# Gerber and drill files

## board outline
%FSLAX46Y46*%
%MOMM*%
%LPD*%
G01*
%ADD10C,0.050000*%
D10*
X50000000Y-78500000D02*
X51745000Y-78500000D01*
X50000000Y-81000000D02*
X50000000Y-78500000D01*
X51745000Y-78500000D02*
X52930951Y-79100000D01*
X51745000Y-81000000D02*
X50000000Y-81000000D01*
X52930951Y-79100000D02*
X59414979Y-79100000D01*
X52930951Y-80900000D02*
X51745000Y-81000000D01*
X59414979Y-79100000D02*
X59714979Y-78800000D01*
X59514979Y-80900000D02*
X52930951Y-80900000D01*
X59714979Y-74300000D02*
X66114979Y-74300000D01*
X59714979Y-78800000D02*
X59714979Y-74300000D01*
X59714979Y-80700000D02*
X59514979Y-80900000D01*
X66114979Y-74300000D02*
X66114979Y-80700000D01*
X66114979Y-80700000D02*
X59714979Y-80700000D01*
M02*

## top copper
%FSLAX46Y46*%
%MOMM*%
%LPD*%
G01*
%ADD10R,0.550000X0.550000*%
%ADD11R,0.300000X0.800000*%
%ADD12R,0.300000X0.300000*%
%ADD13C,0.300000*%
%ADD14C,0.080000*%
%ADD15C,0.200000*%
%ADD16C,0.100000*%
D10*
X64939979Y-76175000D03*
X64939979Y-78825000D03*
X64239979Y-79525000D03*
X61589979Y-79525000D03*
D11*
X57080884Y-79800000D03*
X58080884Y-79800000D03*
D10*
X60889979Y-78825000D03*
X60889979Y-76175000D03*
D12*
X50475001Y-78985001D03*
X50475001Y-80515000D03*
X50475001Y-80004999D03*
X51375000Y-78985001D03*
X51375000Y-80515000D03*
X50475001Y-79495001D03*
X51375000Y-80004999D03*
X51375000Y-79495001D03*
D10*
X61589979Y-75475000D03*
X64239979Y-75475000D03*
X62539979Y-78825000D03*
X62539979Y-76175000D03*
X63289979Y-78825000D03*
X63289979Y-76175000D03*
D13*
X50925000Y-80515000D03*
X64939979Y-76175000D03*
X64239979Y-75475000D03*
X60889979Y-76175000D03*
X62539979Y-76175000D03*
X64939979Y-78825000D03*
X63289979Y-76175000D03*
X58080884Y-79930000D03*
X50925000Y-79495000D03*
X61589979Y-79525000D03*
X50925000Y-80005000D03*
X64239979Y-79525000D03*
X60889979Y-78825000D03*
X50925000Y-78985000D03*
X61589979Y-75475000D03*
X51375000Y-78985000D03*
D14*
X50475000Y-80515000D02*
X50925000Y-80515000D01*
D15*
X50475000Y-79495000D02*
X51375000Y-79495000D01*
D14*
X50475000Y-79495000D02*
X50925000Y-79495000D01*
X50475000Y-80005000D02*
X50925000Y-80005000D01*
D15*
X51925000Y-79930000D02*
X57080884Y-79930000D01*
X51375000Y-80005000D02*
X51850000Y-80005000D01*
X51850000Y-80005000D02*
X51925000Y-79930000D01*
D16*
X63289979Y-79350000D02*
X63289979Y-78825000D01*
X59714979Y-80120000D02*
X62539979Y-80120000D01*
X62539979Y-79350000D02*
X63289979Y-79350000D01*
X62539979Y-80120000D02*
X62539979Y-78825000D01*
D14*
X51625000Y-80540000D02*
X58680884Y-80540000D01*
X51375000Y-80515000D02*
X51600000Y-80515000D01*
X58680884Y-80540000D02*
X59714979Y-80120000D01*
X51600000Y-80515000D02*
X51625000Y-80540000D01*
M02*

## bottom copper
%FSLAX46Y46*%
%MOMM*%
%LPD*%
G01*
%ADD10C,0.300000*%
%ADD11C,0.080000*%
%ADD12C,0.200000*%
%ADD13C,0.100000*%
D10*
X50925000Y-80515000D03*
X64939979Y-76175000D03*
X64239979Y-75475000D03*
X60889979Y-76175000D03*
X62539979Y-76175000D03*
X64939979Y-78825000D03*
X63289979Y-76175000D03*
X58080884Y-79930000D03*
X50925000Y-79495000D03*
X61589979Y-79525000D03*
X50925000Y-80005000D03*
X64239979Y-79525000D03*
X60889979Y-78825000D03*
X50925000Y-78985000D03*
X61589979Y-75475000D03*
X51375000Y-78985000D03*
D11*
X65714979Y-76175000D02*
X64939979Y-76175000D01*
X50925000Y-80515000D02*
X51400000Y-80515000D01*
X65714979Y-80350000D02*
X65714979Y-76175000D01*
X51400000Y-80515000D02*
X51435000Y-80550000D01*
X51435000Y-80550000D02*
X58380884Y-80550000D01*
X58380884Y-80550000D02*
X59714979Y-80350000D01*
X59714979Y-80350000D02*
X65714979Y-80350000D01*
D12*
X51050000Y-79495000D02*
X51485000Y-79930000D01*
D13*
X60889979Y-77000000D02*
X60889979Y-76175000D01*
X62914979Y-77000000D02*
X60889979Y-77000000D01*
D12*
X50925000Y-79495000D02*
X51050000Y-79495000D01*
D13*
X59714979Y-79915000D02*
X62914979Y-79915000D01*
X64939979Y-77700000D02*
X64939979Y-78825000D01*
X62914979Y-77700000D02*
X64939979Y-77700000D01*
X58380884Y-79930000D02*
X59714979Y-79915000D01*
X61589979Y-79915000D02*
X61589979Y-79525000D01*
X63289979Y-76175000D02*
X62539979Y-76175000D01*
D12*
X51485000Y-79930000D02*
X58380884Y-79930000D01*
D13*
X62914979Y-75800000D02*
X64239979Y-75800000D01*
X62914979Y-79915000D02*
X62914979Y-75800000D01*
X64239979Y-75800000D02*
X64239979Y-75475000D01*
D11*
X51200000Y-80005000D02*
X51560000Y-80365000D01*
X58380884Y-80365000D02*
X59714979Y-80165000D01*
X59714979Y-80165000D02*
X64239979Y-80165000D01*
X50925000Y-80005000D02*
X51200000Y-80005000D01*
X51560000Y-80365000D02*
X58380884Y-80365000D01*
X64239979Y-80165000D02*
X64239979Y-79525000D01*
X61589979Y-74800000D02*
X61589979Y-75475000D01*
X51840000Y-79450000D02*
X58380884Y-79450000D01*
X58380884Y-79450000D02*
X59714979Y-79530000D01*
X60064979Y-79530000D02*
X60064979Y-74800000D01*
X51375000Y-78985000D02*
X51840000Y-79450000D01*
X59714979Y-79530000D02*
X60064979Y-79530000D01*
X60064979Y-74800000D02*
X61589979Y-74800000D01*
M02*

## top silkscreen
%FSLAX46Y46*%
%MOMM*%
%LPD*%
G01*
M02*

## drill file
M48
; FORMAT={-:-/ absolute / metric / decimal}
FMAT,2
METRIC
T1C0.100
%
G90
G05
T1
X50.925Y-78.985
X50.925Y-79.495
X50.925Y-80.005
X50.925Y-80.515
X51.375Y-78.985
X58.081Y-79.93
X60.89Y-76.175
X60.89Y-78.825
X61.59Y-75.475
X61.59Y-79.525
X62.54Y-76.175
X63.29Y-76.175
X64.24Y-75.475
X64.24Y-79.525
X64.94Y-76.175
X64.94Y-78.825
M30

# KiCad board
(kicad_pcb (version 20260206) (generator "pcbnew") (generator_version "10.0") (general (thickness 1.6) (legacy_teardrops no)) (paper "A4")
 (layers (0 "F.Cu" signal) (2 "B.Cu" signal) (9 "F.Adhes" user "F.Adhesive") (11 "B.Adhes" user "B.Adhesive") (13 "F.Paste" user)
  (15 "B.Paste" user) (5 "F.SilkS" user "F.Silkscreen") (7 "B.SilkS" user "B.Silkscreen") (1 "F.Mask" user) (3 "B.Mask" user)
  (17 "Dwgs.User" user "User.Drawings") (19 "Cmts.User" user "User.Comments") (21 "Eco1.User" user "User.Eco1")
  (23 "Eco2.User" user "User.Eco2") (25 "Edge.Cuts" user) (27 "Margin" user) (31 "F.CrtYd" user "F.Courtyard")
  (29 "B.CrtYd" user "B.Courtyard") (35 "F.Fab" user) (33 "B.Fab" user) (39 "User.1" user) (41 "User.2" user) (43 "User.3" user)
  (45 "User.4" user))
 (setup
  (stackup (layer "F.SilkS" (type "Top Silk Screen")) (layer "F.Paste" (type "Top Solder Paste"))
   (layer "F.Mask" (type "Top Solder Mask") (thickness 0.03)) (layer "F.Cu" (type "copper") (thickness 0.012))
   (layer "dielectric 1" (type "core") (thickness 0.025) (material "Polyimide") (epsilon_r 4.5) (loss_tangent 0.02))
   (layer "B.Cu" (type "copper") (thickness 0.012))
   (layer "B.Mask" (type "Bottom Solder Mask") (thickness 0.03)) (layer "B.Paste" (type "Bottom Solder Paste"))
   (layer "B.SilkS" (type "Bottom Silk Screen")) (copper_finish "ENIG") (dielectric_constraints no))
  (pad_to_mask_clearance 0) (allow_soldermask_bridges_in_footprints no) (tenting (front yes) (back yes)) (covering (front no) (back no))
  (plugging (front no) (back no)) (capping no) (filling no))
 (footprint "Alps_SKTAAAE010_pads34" (layer "F.Cu") (at 65.314979 77.5 -90)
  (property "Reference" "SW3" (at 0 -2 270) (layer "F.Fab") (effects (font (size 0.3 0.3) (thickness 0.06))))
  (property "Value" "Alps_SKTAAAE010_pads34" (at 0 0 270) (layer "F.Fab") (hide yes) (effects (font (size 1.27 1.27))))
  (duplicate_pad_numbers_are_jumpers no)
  (pad "3" smd rect (at -1.325 0.375 270) (size 0.55 0.55) (layers "F.Cu" "F.Mask") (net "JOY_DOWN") (solder_mask_margin 0.05)
   (thermal_bridge_angle 45))
  (pad "4" smd rect (at 1.325 0.375 270) (size 0.55 0.55) (layers "F.Cu" "F.Mask") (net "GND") (solder_mask_margin 0.05)
   (thermal_bridge_angle 45)))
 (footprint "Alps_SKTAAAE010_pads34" (layer "F.Cu") (at 62.914979 79.9 180)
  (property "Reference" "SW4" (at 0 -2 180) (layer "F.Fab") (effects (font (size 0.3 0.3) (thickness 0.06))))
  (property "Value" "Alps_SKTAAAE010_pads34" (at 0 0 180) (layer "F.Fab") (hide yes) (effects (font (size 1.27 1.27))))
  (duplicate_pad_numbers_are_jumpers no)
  (pad "3" smd rect (at -1.325 0.375 180) (size 0.55 0.55) (layers "F.Cu" "F.Mask") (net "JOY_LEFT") (solder_mask_margin 0.05)
   (thermal_bridge_angle 45))
  (pad "4" smd rect (at 1.325 0.375 180) (size 0.55 0.55) (layers "F.Cu" "F.Mask") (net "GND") (solder_mask_margin 0.05)
   (thermal_bridge_angle 45)))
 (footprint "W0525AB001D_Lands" (layer "F.Cu") (at 57.580884 79.93)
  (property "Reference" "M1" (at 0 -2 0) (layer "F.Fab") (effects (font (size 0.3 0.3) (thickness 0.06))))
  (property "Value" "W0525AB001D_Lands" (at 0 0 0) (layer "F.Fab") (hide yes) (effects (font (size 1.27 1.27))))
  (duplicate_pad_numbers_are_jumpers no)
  (pad "1" smd rect (at -0.5 -0.13) (size 0.3 0.8) (layers "F.Cu" "F.Mask") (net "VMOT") (solder_mask_margin 0.05) (thermal_bridge_angle 45))
  (pad "2" smd rect (at 0.5 -0.13) (size 0.3 0.8) (layers "F.Cu" "F.Mask") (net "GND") (solder_mask_margin 0.05) (thermal_bridge_angle 45)))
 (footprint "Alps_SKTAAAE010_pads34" (layer "F.Cu") (at 60.514979 77.5 90)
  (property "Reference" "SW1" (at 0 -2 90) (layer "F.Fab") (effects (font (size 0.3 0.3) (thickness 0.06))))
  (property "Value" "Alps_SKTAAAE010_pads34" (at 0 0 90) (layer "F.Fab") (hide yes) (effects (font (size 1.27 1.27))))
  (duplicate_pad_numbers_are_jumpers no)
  (pad "3" smd rect (at -1.325 0.375 90) (size 0.55 0.55) (layers "F.Cu" "F.Mask") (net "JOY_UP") (solder_mask_margin 0.05)
   (thermal_bridge_angle 45))
  (pad "4" smd rect (at 1.325 0.375 90) (size 0.55 0.55) (layers "F.Cu" "F.Mask") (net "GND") (solder_mask_margin 0.05)
   (thermal_bridge_angle 45)))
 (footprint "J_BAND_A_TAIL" (layer "F.Cu") (at 50.9 79.75)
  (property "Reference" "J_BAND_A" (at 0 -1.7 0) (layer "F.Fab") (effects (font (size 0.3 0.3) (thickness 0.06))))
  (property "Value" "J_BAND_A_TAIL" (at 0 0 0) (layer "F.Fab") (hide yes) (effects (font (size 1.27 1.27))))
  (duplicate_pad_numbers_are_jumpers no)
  (pad "1" smd rect (at -0.424999 -0.764999) (size 0.3 0.3) (layers "F.Cu" "F.Mask") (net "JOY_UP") (solder_mask_margin 0.05)
   (thermal_bridge_angle 45))
  (pad "2" smd rect (at -0.424999 0.765) (size 0.3 0.3) (layers "F.Cu" "F.Mask") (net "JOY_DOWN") (solder_mask_margin 0.05)
   (thermal_bridge_angle 45))
  (pad "3" smd rect (at -0.424999 0.254999) (size 0.3 0.3) (layers "F.Cu" "F.Mask") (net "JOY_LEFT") (solder_mask_margin 0.05)
   (thermal_bridge_angle 45))
  (pad "4" smd rect (at 0.475 -0.764999) (size 0.3 0.3) (layers "F.Cu" "F.Mask") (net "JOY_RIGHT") (solder_mask_margin 0.05)
   (thermal_bridge_angle 45))
  (pad "5" smd rect (at 0.475 0.765) (size 0.3 0.3) (layers "F.Cu" "F.Mask") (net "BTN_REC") (solder_mask_margin 0.05)
   (thermal_bridge_angle 45))
  (pad "6" smd rect (at -0.424999 -0.254999) (size 0.3 0.3) (layers "F.Cu" "F.Mask") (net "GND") (solder_mask_margin 0.05)
   (thermal_bridge_angle 45))
  (pad "7" smd rect (at 0.475 0.254999) (size 0.3 0.3) (layers "F.Cu" "F.Mask") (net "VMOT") (solder_mask_margin 0.05)
   (thermal_bridge_angle 45))
  (pad "8" smd rect (at 0.475 -0.254999) (size 0.3 0.3) (layers "F.Cu" "F.Mask") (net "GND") (solder_mask_margin 0.05)
   (thermal_bridge_angle 45)))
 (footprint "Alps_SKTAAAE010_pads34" (layer "F.Cu") (at 62.914979 75.1)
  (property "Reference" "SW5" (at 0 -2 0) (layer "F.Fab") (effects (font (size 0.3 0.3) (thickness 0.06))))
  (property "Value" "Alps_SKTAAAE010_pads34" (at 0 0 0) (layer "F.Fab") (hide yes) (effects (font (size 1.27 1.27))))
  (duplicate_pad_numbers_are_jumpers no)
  (pad "3" smd rect (at -1.325 0.375) (size 0.55 0.55) (layers "F.Cu" "F.Mask") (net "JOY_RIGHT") (solder_mask_margin 0.05)
   (thermal_bridge_angle 45))
  (pad "4" smd rect (at 1.325 0.375) (size 0.55 0.55) (layers "F.Cu" "F.Mask") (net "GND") (solder_mask_margin 0.05)
   (thermal_bridge_angle 45)))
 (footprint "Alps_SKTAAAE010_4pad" (layer "F.Cu") (at 62.914979 77.5 90)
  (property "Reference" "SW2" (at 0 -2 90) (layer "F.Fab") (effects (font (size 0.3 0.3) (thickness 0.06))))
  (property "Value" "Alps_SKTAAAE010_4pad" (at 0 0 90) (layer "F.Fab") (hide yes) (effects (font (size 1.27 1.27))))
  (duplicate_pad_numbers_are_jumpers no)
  (pad "1" smd rect (at -1.325 -0.375 90) (size 0.55 0.55) (layers "F.Cu" "F.Mask") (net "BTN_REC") (solder_mask_margin 0.05)
   (thermal_bridge_angle 45))
  (pad "2" smd rect (at 1.325 -0.375 90) (size 0.55 0.55) (layers "F.Cu" "F.Mask") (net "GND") (solder_mask_margin 0.05)
   (thermal_bridge_angle 45))
  (pad "3" smd rect (at -1.325 0.375 90) (size 0.55 0.55) (layers "F.Cu" "F.Mask") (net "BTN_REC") (solder_mask_margin 0.05)
   (thermal_bridge_angle 45))
  (pad "4" smd rect (at 1.325 0.375 90) (size 0.55 0.55) (layers "F.Cu" "F.Mask") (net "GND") (solder_mask_margin 0.05)
   (thermal_bridge_angle 45)))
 (gr_line (start 50 78.5) (end 51.745 78.5) (stroke (width 0.05) (type default)) (layer "Edge.Cuts"))
 (gr_line (start 50 81) (end 50 78.5) (stroke (width 0.05) (type default)) (layer "Edge.Cuts"))
 (gr_line (start 51.745 78.5) (end 52.930951 79.1) (stroke (width 0.05) (type default)) (layer "Edge.Cuts"))
 (gr_line (start 51.745 81) (end 50 81) (stroke (width 0.05) (type default)) (layer "Edge.Cuts"))
 (gr_line (start 52.930951 79.1) (end 59.414979 79.1) (stroke (width 0.05) (type default)) (layer "Edge.Cuts"))
 (gr_line (start 52.930951 80.9) (end 51.745 81) (stroke (width 0.05) (type default)) (layer "Edge.Cuts"))
 (gr_line (start 59.414979 79.1) (end 59.714979 78.8) (stroke (width 0.05) (type default)) (layer "Edge.Cuts"))
 (gr_line (start 59.514979 80.9) (end 52.930951 80.9) (stroke (width 0.05) (type default)) (layer "Edge.Cuts"))
 (gr_line (start 59.714979 74.3) (end 66.114979 74.3) (stroke (width 0.05) (type default)) (layer "Edge.Cuts"))
 (gr_line (start 59.714979 78.8) (end 59.714979 74.3) (stroke (width 0.05) (type default)) (layer "Edge.Cuts"))
 (gr_line (start 59.714979 80.7) (end 59.514979 80.9) (stroke (width 0.05) (type default)) (layer "Edge.Cuts"))
 (gr_line (start 66.114979 74.3) (end 66.114979 80.7) (stroke (width 0.05) (type default)) (layer "Edge.Cuts"))
 (gr_line (start 66.114979 80.7) (end 59.714979 80.7) (stroke (width 0.05) (type default)) (layer "Edge.Cuts"))
 (segment (start 50.475 80.515) (end 50.925 80.515) (width 0.08) (layer "F.Cu") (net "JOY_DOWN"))
 (via (at 50.925 80.515) (size 0.3) (drill 0.1) (layers "F.Cu" "B.Cu") (tenting (front yes) (back yes)) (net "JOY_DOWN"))
 (via (at 64.939979 76.175) (size 0.3) (drill 0.1) (layers "F.Cu" "B.Cu") (tenting (front yes) (back yes)) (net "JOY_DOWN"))
 (segment (start 65.714979 76.175) (end 64.939979 76.175) (width 0.08) (layer "B.Cu") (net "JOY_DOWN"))
 (segment (start 50.925 80.515) (end 51.4 80.515) (width 0.08) (layer "B.Cu") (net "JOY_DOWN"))
 (segment (start 65.714979 80.35) (end 65.714979 76.175) (width 0.08) (layer "B.Cu") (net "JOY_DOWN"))
 (segment (start 51.4 80.515) (end 51.435 80.55) (width 0.08) (layer "B.Cu") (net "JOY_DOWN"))
 (segment (start 51.435 80.55) (end 58.380884 80.55) (width 0.08) (layer "B.Cu") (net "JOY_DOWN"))
 (segment (start 58.380884 80.55) (end 59.714979 80.35) (width 0.08) (layer "B.Cu") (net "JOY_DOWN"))
 (segment (start 59.714979 80.35) (end 65.714979 80.35) (width 0.08) (layer "B.Cu") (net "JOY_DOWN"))
 (segment (start 50.475 79.495) (end 51.375 79.495) (width 0.2) (layer "F.Cu") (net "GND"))
 (segment (start 50.475 79.495) (end 50.925 79.495) (width 0.08) (layer "F.Cu") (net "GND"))
 (via (at 64.239979 75.475) (size 0.3) (drill 0.1) (layers "F.Cu" "B.Cu") (tenting (front yes) (back yes)) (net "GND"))
 (via (at 60.889979 76.175) (size 0.3) (drill 0.1) (layers "F.Cu" "B.Cu") (tenting (front yes) (back yes)) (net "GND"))
 (via (at 62.539979 76.175) (size 0.3) (drill 0.1) (layers "F.Cu" "B.Cu") (tenting (front yes) (back yes)) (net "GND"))
 (via (at 64.939979 78.825) (size 0.3) (drill 0.1) (layers "F.Cu" "B.Cu") (tenting (front yes) (back yes)) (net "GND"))
 (via (at 63.289979 76.175) (size 0.3) (drill 0.1) (layers "F.Cu" "B.Cu") (tenting (front yes) (back yes)) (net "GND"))
 (via (at 58.080884 79.93) (size 0.3) (drill 0.1) (layers "F.Cu" "B.Cu") (tenting (front yes) (back yes)) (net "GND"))
 (via (at 50.925 79.495) (size 0.3) (drill 0.1) (layers "F.Cu" "B.Cu") (tenting (front yes) (back yes)) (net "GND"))
 (via (at 61.589979 79.525) (size 0.3) (drill 0.1) (layers "F.Cu" "B.Cu") (tenting (front yes) (back yes)) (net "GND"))
 (segment (start 51.05 79.495) (end 51.485 79.93) (width 0.2) (layer "B.Cu") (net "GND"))
 (segment (start 60.889979 77) (end 60.889979 76.175) (width 0.1) (layer "B.Cu") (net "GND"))
 (segment (start 62.914979 77) (end 60.889979 77) (width 0.1) (layer "B.Cu") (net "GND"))
 (segment (start 50.925 79.495) (end 51.05 79.495) (width 0.2) (layer "B.Cu") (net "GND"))
 (segment (start 59.714979 79.915) (end 62.914979 79.915) (width 0.1) (layer "B.Cu") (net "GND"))
 (segment (start 64.939979 77.7) (end 64.939979 78.825) (width 0.1) (layer "B.Cu") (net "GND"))
 (segment (start 62.914979 77.7) (end 64.939979 77.7) (width 0.1) (layer "B.Cu") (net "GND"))
 (segment (start 58.380884 79.93) (end 59.714979 79.915) (width 0.1) (layer "B.Cu") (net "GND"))
 (segment (start 61.589979 79.915) (end 61.589979 79.525) (width 0.1) (layer "B.Cu") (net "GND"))
 (segment (start 63.289979 76.175) (end 62.539979 76.175) (width 0.1) (layer "B.Cu") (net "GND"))
 (segment (start 51.485 79.93) (end 58.380884 79.93) (width 0.2) (layer "B.Cu") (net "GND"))
 (segment (start 62.914979 75.8) (end 64.239979 75.8) (width 0.1) (layer "B.Cu") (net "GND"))
 (segment (start 62.914979 79.915) (end 62.914979 75.8) (width 0.1) (layer "B.Cu") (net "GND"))
 (segment (start 64.239979 75.8) (end 64.239979 75.475) (width 0.1) (layer "B.Cu") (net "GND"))
 (segment (start 50.475 80.005) (end 50.925 80.005) (width 0.08) (layer "F.Cu") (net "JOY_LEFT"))
 (via (at 50.925 80.005) (size 0.3) (drill 0.1) (layers "F.Cu" "B.Cu") (tenting (front yes) (back yes)) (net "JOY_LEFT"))
 (via (at 64.239979 79.525) (size 0.3) (drill 0.1) (layers "F.Cu" "B.Cu") (tenting (front yes) (back yes)) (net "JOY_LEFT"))
 (segment (start 51.2 80.005) (end 51.56 80.365) (width 0.08) (layer "B.Cu") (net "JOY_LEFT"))
 (segment (start 58.380884 80.365) (end 59.714979 80.165) (width 0.08) (layer "B.Cu") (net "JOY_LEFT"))
 (segment (start 59.714979 80.165) (end 64.239979 80.165) (width 0.08) (layer "B.Cu") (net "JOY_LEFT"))
 (segment (start 50.925 80.005) (end 51.2 80.005) (width 0.08) (layer "B.Cu") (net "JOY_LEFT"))
 (segment (start 51.56 80.365) (end 58.380884 80.365) (width 0.08) (layer "B.Cu") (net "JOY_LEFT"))
 (segment (start 64.239979 80.165) (end 64.239979 79.525) (width 0.08) (layer "B.Cu") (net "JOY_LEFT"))
 (segment (start 51.925 79.93) (end 57.080884 79.93) (width 0.2) (layer "F.Cu") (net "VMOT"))
 (segment (start 51.375 80.005) (end 51.85 80.005) (width 0.2) (layer "F.Cu") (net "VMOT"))
 (segment (start 51.85 80.005) (end 51.925 79.93) (width 0.2) (layer "F.Cu") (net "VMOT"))
 (via (at 60.889979 78.825) (size 0.3) (drill 0.1) (layers "F.Cu" "B.Cu") (tenting (front yes) (back yes)) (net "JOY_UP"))
 (via (at 50.925 78.985) (size 0.3) (drill 0.1) (layers "F.Cu" "B.Cu") (tenting (front yes) (back yes)) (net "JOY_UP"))
 (via (at 61.589979 75.475) (size 0.3) (drill 0.1) (layers "F.Cu" "B.Cu") (tenting (front yes) (back yes)) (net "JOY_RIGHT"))
 (via (at 51.375 78.985) (size 0.3) (drill 0.1) (layers "F.Cu" "B.Cu") (tenting (front yes) (back yes)) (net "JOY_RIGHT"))
 (segment (start 61.589979 74.8) (end 61.589979 75.475) (width 0.08) (layer "B.Cu") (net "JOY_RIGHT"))
 (segment (start 51.84 79.45) (end 58.380884 79.45) (width 0.08) (layer "B.Cu") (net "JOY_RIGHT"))
 (segment (start 58.380884 79.45) (end 59.714979 79.53) (width 0.08) (layer "B.Cu") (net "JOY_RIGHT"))
 (segment (start 60.064979 79.53) (end 60.064979 74.8) (width 0.08) (layer "B.Cu") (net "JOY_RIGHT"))
 (segment (start 51.375 78.985) (end 51.84 79.45) (width 0.08) (layer "B.Cu") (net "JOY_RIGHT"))
 (segment (start 59.714979 79.53) (end 60.064979 79.53) (width 0.08) (layer "B.Cu") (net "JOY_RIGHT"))
 (segment (start 60.064979 74.8) (end 61.589979 74.8) (width 0.08) (layer "B.Cu") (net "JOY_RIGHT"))
 (segment (start 63.289979 79.35) (end 63.289979 78.825) (width 0.1) (layer "F.Cu") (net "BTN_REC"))
 (segment (start 59.714979 80.12) (end 62.539979 80.12) (width 0.1) (layer "F.Cu") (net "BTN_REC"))
 (segment (start 62.539979 79.35) (end 63.289979 79.35) (width 0.1) (layer "F.Cu") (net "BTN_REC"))
 (segment (start 62.539979 80.12) (end 62.539979 78.825) (width 0.1) (layer "F.Cu") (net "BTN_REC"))
 (segment (start 51.625 80.54) (end 58.680884 80.54) (width 0.08) (layer "F.Cu") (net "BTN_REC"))
 (segment (start 51.375 80.515) (end 51.6 80.515) (width 0.08) (layer "F.Cu") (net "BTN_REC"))
 (segment (start 58.680884 80.54) (end 59.714979 80.12) (width 0.08) (layer "F.Cu") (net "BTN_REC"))
 (segment (start 51.6 80.515) (end 51.625 80.54) (width 0.08) (layer "F.Cu") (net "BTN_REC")))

